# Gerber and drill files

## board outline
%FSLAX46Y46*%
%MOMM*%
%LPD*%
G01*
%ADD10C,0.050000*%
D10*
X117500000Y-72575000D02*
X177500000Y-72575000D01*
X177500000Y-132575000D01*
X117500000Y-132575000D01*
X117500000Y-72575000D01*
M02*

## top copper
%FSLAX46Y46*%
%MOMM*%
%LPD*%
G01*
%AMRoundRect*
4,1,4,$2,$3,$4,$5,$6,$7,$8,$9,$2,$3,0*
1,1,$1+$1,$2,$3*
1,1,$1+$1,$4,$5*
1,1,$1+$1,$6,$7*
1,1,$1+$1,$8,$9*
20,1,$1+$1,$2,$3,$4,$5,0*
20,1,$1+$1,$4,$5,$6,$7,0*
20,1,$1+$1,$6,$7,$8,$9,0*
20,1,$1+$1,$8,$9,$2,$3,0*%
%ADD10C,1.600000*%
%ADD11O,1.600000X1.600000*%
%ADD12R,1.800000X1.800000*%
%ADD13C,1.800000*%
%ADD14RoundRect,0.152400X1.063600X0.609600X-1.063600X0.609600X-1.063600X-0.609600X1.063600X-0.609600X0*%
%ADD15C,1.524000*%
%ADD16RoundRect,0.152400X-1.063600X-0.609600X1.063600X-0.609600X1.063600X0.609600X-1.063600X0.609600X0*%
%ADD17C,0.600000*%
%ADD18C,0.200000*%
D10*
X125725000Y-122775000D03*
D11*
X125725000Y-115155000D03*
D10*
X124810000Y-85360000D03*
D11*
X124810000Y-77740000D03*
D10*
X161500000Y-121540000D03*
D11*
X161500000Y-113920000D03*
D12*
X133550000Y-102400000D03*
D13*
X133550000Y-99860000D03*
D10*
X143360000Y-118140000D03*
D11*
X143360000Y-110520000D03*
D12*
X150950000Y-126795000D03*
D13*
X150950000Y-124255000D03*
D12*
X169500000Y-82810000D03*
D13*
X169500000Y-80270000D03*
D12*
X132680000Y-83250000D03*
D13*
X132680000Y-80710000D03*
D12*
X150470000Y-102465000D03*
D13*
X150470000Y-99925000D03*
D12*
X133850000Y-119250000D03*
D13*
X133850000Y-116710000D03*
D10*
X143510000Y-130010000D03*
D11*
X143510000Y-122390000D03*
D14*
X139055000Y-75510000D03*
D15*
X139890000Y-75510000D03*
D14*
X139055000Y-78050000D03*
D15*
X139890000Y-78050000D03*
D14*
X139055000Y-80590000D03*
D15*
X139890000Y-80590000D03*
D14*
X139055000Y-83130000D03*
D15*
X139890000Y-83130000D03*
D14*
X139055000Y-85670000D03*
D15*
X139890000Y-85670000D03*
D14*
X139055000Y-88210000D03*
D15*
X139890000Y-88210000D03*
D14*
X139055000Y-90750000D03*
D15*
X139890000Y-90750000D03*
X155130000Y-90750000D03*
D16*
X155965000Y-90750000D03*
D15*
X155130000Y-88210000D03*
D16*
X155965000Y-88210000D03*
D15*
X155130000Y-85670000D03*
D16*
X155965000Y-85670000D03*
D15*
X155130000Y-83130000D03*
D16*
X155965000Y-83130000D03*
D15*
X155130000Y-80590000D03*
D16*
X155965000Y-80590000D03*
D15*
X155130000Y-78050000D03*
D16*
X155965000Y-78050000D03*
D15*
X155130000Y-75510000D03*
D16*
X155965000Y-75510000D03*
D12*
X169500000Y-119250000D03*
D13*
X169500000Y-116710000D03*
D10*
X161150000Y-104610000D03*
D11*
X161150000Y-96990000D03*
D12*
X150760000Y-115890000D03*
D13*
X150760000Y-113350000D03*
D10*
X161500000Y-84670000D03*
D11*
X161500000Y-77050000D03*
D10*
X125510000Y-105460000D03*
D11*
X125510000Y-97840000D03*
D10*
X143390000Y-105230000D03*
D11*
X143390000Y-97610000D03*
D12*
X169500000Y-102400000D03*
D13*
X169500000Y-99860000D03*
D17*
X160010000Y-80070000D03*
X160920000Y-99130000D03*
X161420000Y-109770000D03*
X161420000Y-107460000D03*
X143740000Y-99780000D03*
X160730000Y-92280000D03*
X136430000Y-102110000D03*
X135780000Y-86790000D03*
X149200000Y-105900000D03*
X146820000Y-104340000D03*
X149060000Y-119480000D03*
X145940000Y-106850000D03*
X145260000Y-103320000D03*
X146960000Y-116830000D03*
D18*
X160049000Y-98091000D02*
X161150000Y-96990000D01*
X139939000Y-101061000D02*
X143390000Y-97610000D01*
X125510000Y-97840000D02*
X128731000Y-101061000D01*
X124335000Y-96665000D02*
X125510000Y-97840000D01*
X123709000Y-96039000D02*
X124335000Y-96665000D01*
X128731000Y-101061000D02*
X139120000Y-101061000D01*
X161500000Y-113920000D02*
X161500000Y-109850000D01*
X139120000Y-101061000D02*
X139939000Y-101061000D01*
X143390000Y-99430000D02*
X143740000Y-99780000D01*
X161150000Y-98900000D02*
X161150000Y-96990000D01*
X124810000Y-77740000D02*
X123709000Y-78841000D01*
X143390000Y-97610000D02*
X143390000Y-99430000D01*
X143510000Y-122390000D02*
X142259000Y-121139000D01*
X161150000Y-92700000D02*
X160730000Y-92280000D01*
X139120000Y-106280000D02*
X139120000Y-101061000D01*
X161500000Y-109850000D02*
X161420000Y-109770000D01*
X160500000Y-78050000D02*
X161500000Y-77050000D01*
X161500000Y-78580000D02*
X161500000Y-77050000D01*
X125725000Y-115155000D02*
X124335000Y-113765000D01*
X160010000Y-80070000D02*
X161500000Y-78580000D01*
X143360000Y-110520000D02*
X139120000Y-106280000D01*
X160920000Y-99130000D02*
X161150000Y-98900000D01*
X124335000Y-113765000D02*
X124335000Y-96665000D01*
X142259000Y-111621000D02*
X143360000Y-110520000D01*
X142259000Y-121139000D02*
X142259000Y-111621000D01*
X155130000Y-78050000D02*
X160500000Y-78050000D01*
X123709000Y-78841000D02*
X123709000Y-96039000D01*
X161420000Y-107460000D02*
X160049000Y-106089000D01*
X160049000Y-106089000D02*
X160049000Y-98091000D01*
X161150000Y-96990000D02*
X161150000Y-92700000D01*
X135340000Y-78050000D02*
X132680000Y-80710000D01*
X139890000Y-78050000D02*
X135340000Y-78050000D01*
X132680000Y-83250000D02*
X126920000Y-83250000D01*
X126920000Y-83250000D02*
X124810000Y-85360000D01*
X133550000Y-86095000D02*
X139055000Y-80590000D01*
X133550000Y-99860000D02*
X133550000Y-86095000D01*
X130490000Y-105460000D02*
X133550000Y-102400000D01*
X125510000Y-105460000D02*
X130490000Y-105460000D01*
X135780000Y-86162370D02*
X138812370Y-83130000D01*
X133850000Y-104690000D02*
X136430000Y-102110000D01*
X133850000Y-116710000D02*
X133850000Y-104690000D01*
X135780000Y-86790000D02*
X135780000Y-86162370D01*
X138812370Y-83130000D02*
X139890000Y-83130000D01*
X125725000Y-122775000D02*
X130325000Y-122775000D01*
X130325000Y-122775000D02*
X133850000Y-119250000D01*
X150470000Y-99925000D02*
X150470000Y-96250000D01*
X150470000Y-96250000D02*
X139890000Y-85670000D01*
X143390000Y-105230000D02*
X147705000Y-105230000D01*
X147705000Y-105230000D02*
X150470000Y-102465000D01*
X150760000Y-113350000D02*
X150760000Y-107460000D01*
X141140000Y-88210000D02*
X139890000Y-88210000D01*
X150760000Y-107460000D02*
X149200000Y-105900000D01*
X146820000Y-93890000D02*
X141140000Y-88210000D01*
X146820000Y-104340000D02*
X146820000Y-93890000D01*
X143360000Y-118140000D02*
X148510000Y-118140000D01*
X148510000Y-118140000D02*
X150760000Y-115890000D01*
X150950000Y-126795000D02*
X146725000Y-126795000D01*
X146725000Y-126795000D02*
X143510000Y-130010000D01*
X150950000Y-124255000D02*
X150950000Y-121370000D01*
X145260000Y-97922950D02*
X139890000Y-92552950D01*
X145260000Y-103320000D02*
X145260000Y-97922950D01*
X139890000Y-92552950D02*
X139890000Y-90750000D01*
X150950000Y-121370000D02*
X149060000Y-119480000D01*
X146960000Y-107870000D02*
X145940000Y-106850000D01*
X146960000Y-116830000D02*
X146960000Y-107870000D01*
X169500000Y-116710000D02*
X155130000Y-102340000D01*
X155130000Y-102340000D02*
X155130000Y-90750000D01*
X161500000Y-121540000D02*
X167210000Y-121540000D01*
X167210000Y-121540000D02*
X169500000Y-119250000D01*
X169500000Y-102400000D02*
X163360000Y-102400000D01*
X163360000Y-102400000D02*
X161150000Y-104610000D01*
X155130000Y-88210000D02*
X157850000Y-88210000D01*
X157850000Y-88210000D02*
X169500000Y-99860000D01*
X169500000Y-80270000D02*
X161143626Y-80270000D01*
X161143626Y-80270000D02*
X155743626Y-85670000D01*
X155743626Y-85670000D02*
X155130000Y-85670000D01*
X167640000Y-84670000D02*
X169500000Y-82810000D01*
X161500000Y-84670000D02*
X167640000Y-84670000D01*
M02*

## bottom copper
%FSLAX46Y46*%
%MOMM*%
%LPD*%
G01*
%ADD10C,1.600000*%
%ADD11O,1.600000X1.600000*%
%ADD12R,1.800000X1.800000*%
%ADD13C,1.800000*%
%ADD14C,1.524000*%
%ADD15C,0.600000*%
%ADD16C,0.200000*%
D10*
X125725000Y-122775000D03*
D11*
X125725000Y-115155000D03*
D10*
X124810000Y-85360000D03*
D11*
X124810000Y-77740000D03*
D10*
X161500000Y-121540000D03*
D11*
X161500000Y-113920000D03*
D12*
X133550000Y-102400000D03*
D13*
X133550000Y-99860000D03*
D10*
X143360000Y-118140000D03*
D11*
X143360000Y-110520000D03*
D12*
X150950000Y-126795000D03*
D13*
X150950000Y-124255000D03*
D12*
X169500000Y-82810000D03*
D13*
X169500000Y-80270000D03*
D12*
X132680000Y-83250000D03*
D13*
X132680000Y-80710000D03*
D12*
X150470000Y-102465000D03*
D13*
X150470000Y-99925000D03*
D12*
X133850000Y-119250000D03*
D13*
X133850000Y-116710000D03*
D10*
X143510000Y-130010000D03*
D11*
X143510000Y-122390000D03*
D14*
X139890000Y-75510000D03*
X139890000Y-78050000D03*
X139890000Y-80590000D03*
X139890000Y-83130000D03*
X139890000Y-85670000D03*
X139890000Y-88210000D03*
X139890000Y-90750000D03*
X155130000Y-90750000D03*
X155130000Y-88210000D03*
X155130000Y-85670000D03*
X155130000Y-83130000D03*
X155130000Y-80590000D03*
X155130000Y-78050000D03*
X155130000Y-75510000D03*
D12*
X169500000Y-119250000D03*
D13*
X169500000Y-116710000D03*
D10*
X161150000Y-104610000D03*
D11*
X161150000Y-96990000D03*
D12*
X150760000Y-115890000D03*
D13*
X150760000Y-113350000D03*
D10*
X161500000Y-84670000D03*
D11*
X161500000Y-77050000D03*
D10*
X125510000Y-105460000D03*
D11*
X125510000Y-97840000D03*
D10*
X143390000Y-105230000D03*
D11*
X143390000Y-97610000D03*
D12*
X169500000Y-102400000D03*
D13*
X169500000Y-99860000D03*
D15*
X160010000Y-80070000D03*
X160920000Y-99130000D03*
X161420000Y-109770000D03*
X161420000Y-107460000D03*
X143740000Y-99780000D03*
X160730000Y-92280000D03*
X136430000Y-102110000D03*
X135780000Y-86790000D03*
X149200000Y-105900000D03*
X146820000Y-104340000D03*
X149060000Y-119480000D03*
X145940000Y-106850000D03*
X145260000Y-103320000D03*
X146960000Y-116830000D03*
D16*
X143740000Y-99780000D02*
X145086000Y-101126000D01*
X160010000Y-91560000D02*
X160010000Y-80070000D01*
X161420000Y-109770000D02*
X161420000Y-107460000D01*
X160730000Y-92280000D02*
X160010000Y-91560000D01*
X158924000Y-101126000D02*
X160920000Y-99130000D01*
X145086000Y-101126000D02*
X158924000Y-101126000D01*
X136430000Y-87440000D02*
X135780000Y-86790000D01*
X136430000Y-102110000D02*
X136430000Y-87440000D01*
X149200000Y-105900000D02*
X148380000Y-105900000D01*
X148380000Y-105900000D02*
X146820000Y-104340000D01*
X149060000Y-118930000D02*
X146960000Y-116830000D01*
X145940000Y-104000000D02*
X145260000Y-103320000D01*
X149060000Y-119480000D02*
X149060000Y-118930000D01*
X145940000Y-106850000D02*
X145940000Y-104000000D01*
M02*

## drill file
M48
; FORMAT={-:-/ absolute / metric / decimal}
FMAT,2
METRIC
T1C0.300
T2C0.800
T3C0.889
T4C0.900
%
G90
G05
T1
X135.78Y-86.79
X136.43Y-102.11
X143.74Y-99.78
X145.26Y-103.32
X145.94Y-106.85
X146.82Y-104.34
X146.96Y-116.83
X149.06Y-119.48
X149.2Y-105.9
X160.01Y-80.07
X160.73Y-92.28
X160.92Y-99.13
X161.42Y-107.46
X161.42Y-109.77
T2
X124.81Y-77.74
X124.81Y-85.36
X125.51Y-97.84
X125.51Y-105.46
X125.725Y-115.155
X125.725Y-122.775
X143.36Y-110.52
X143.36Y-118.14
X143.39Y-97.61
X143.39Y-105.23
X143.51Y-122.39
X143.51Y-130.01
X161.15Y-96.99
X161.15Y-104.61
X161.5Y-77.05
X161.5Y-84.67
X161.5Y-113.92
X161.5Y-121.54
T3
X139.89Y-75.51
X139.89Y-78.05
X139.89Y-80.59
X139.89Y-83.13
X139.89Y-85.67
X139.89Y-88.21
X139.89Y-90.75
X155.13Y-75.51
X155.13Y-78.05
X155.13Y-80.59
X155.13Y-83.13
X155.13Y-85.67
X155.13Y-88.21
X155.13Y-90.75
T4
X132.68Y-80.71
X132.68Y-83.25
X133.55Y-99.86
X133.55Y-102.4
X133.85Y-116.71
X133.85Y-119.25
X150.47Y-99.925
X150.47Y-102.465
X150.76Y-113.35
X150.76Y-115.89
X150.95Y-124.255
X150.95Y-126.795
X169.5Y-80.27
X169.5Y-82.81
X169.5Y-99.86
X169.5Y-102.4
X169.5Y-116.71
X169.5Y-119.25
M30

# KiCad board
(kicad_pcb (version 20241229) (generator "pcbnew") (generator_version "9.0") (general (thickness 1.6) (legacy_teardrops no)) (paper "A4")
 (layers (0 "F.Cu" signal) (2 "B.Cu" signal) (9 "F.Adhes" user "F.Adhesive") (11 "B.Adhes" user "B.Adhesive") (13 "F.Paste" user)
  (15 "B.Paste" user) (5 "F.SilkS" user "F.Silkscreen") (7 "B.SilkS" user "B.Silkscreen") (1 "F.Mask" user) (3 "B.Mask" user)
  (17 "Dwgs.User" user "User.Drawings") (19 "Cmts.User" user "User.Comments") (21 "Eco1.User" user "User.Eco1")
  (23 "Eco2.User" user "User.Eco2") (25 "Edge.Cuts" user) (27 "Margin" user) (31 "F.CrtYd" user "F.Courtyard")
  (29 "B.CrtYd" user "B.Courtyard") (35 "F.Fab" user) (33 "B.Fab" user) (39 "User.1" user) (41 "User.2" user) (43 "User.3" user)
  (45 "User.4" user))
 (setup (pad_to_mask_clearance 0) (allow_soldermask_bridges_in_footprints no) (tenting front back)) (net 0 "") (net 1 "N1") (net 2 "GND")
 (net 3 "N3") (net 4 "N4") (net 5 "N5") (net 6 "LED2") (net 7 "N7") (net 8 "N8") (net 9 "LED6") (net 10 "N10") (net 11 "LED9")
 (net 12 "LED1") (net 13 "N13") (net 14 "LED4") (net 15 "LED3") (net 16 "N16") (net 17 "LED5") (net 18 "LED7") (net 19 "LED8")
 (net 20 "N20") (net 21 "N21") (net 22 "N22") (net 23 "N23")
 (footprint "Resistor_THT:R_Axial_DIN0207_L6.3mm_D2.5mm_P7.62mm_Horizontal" (layer "F.Cu") (at 125.725 122.775 90)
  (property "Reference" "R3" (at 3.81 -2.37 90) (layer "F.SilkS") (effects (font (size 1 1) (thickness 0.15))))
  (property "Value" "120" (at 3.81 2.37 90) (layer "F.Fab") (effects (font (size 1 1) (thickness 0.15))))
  (pad "1" thru_hole circle (at 0 0 90) (size 1.6 1.6) (drill 0.8) (layers "*.Cu" "*.Mask") (remove_unused_layers no) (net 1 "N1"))
  (pad "2" thru_hole oval (at 7.62 0 90) (size 1.6 1.6) (drill 0.8) (layers "*.Cu" "*.Mask") (remove_unused_layers no) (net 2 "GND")))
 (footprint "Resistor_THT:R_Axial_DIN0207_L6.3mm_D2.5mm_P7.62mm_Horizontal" (layer "F.Cu") (at 124.81 85.36 90)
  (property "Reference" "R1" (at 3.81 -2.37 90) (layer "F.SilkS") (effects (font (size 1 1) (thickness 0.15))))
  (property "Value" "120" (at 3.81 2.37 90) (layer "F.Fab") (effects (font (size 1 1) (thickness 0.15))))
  (pad "1" thru_hole circle (at 0 0 90) (size 1.6 1.6) (drill 0.8) (layers "*.Cu" "*.Mask") (remove_unused_layers no) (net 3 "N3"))
  (pad "2" thru_hole oval (at 7.62 0 90) (size 1.6 1.6) (drill 0.8) (layers "*.Cu" "*.Mask") (remove_unused_layers no) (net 2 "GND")))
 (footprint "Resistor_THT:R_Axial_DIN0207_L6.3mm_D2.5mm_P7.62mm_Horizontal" (layer "F.Cu") (at 161.5 121.54 90)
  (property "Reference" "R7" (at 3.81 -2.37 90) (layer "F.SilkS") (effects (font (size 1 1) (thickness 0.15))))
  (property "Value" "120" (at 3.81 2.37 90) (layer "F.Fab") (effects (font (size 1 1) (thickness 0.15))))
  (pad "1" thru_hole circle (at 0 0 90) (size 1.6 1.6) (drill 0.8) (layers "*.Cu" "*.Mask") (remove_unused_layers no) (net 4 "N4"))
  (pad "2" thru_hole oval (at 7.62 0 90) (size 1.6 1.6) (drill 0.8) (layers "*.Cu" "*.Mask") (remove_unused_layers no) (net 2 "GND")))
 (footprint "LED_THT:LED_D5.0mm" (layer "F.Cu") (at 133.55 102.4 90)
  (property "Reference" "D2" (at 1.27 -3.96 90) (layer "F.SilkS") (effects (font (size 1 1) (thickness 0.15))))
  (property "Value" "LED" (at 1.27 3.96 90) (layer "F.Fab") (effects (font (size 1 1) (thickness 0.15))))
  (pad "1" thru_hole rect (at 0 0 90) (size 1.8 1.8) (drill 0.9) (layers "*.Cu" "*.Mask") (remove_unused_layers no) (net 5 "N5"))
  (pad "2" thru_hole circle (at 2.54 0 90) (size 1.8 1.8) (drill 0.9) (layers "*.Cu" "*.Mask") (remove_unused_layers no) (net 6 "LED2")))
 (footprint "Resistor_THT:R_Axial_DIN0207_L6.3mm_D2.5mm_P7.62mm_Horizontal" (layer "F.Cu") (at 143.36 118.14 90)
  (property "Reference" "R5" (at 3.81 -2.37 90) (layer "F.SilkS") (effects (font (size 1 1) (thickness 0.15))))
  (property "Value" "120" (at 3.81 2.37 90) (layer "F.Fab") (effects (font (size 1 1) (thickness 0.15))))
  (pad "1" thru_hole circle (at 0 0 90) (size 1.6 1.6) (drill 0.8) (layers "*.Cu" "*.Mask") (remove_unused_layers no) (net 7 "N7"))
  (pad "2" thru_hole oval (at 7.62 0 90) (size 1.6 1.6) (drill 0.8) (layers "*.Cu" "*.Mask") (remove_unused_layers no) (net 2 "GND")))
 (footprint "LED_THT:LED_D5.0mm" (layer "F.Cu") (at 150.95 126.795 90)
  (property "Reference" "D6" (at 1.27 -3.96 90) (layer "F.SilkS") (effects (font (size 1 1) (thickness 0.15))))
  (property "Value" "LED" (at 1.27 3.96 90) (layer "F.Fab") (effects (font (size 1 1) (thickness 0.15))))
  (pad "1" thru_hole rect (at 0 0 90) (size 1.8 1.8) (drill 0.9) (layers "*.Cu" "*.Mask") (remove_unused_layers no) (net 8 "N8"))
  (pad "2" thru_hole circle (at 2.54 0 90) (size 1.8 1.8) (drill 0.9) (layers "*.Cu" "*.Mask") (remove_unused_layers no) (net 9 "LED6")))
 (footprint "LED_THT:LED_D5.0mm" (layer "F.Cu") (at 169.5 82.81 90)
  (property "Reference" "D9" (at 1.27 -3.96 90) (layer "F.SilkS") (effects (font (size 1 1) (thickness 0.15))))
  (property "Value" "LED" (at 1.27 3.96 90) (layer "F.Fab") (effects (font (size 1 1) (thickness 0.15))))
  (pad "1" thru_hole rect (at 0 0 90) (size 1.8 1.8) (drill 0.9) (layers "*.Cu" "*.Mask") (remove_unused_layers no) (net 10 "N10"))
  (pad "2" thru_hole circle (at 2.54 0 90) (size 1.8 1.8) (drill 0.9) (layers "*.Cu" "*.Mask") (remove_unused_layers no) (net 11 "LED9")))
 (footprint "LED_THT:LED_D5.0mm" (layer "F.Cu") (at 132.68 83.25 90)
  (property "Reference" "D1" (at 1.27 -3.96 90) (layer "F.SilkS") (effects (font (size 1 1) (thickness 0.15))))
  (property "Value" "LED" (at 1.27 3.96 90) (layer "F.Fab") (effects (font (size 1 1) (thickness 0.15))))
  (pad "1" thru_hole rect (at 0 0 90) (size 1.8 1.8) (drill 0.9) (layers "*.Cu" "*.Mask") (remove_unused_layers no) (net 3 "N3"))
  (pad "2" thru_hole circle (at 2.54 0 90) (size 1.8 1.8) (drill 0.9) (layers "*.Cu" "*.Mask") (remove_unused_layers no) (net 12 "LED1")))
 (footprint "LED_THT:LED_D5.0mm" (layer "F.Cu") (at 150.47 102.465 90)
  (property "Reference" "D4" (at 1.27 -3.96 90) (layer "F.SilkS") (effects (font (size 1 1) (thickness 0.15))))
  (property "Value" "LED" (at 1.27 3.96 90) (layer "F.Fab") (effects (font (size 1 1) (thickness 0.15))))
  (pad "1" thru_hole rect (at 0 0 90) (size 1.8 1.8) (drill 0.9) (layers "*.Cu" "*.Mask") (remove_unused_layers no) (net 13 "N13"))
  (pad "2" thru_hole circle (at 2.54 0 90) (size 1.8 1.8) (drill 0.9) (layers "*.Cu" "*.Mask") (remove_unused_layers no) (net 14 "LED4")))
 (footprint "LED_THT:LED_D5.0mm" (layer "F.Cu") (at 133.85 119.25 90)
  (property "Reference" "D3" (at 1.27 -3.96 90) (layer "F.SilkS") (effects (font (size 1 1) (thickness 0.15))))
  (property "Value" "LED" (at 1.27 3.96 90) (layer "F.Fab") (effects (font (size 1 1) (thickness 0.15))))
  (pad "1" thru_hole rect (at 0 0 90) (size 1.8 1.8) (drill 0.9) (layers "*.Cu" "*.Mask") (remove_unused_layers no) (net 1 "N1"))
  (pad "2" thru_hole circle (at 2.54 0 90) (size 1.8 1.8) (drill 0.9) (layers "*.Cu" "*.Mask") (remove_unused_layers no) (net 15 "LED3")))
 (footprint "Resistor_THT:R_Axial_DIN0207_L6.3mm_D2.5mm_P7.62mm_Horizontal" (layer "F.Cu") (at 143.51 130.01 90)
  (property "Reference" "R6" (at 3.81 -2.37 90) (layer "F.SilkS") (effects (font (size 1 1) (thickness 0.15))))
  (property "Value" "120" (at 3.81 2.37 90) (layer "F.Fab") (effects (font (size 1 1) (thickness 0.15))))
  (pad "1" thru_hole circle (at 0 0 90) (size 1.6 1.6) (drill 0.8) (layers "*.Cu" "*.Mask") (remove_unused_layers no) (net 8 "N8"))
  (pad "2" thru_hole oval (at 7.62 0 90) (size 1.6 1.6) (drill 0.8) (layers "*.Cu" "*.Mask") (remove_unused_layers no) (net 2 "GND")))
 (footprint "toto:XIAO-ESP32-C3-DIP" (layer "F.Cu") (at 147.51 83.13 90)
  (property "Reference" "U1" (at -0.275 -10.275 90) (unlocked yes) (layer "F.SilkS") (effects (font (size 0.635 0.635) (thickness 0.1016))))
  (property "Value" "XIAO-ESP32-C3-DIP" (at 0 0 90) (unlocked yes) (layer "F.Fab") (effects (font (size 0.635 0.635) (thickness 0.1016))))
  (pad "1" smd roundrect (at 7.62 -8.455 180) (size 2.432 1.524) (layers "F.Cu" "F.Mask") (roundrect_rratio 0.1) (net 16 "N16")
   (thermal_bridge_angle 45))
  (pad "1" thru_hole circle (at 7.62 -7.62 180) (size 1.524 1.524) (drill 0.889) (layers "*.Cu" "*.Mask") (remove_unused_layers no)
   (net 16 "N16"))
  (pad "2" smd roundrect (at 5.08 -8.455 180) (size 2.432 1.524) (layers "F.Cu" "F.Mask") (roundrect_rratio 0.1) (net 12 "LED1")
   (thermal_bridge_angle 45))
  (pad "2" thru_hole circle (at 5.08 -7.62 180) (size 1.524 1.524) (drill 0.889) (layers "*.Cu" "*.Mask") (remove_unused_layers no)
   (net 12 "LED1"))
  (pad "3" smd roundrect (at 2.54 -8.455 180) (size 2.432 1.524) (layers "F.Cu" "F.Mask") (roundrect_rratio 0.1) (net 6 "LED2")
   (thermal_bridge_angle 45))
  (pad "3" thru_hole circle (at 2.54 -7.62 180) (size 1.524 1.524) (drill 0.889) (layers "*.Cu" "*.Mask") (remove_unused_layers no)
   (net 6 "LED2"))
  (pad "4" smd roundrect (at 0 -8.455 180) (size 2.432 1.524) (layers "F.Cu" "F.Mask") (roundrect_rratio 0.1) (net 15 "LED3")
   (thermal_bridge_angle 45))
  (pad "4" thru_hole circle (at 0 -7.62 180) (size 1.524 1.524) (drill 0.889) (layers "*.Cu" "*.Mask") (remove_unused_layers no)
   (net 15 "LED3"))
  (pad "5" smd roundrect (at -2.54 -8.455 180) (size 2.432 1.524) (layers "F.Cu" "F.Mask") (roundrect_rratio 0.1) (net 14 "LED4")
   (thermal_bridge_angle 45))
  (pad "5" thru_hole circle (at -2.54 -7.62 180) (size 1.524 1.524) (drill 0.889) (layers "*.Cu" "*.Mask") (remove_unused_layers no)
   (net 14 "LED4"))
  (pad "6" smd roundrect (at -5.08 -8.455 180) (size 2.432 1.524) (layers "F.Cu" "F.Mask") (roundrect_rratio 0.1) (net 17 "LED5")
   (thermal_bridge_angle 45))
  (pad "6" thru_hole circle (at -5.08 -7.62 180) (size 1.524 1.524) (drill 0.889) (layers "*.Cu" "*.Mask") (remove_unused_layers no)
   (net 17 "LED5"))
  (pad "7" smd roundrect (at -7.62 -8.455 180) (size 2.432 1.524) (layers "F.Cu" "F.Mask") (roundrect_rratio 0.1) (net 9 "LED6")
   (thermal_bridge_angle 45))
  (pad "7" thru_hole circle (at -7.62 -7.62 180) (size 1.524 1.524) (drill 0.889) (layers "*.Cu" "*.Mask") (remove_unused_layers no)
   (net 9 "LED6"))
  (pad "8" thru_hole circle (at -7.62 7.62) (size 1.524 1.524) (drill 0.889) (layers "*.Cu" "*.Mask") (remove_unused_layers no)
   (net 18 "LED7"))
  (pad "8" smd roundrect (at -7.62 8.455) (size 2.432 1.524) (layers "F.Cu" "F.Mask") (roundrect_rratio 0.1) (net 18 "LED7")
   (thermal_bridge_angle 45))
  (pad "9" thru_hole circle (at -5.08 7.62) (size 1.524 1.524) (drill 0.889) (layers "*.Cu" "*.Mask") (remove_unused_layers no)
   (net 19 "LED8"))
  (pad "9" smd roundrect (at -5.08 8.455) (size 2.432 1.524) (layers "F.Cu" "F.Mask") (roundrect_rratio 0.1) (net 19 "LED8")
   (thermal_bridge_angle 45))
  (pad "10" thru_hole circle (at -2.54 7.62) (size 1.524 1.524) (drill 0.889) (layers "*.Cu" "*.Mask") (remove_unused_layers no)
   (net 11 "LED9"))
  (pad "10" smd roundrect (at -2.54 8.455) (size 2.432 1.524) (layers "F.Cu" "F.Mask") (roundrect_rratio 0.1) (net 11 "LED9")
   (thermal_bridge_angle 45))
  (pad "11" thru_hole circle (at 0 7.62) (size 1.524 1.524) (drill 0.889) (layers "*.Cu" "*.Mask") (remove_unused_layers no) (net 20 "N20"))
  (pad "11" smd roundrect (at 0 8.455) (size 2.432 1.524) (layers "F.Cu" "F.Mask") (roundrect_rratio 0.1) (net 20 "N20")
   (thermal_bridge_angle 45))
  (pad "12" thru_hole circle (at 2.54 7.62) (size 1.524 1.524) (drill 0.889) (layers "*.Cu" "*.Mask") (remove_unused_layers no)
   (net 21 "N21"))
  (pad "12" smd roundrect (at 2.54 8.455) (size 2.432 1.524) (layers "F.Cu" "F.Mask") (roundrect_rratio 0.1) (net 21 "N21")
   (thermal_bridge_angle 45))
  (pad "13" thru_hole circle (at 5.08 7.62) (size 1.524 1.524) (drill 0.889) (layers "*.Cu" "*.Mask") (remove_unused_layers no)
   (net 2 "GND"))
  (pad "13" smd roundrect (at 5.08 8.455) (size 2.432 1.524) (layers "F.Cu" "F.Mask") (roundrect_rratio 0.1) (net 2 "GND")
   (thermal_bridge_angle 45))
  (pad "14" thru_hole circle (at 7.62 7.62) (size 1.524 1.524) (drill 0.889) (layers "*.Cu" "*.Mask") (remove_unused_layers no)
   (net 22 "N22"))
  (pad "14" smd roundrect (at 7.62 8.455) (size 2.432 1.524) (layers "F.Cu" "F.Mask") (roundrect_rratio 0.1) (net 22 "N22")
   (thermal_bridge_angle 45)))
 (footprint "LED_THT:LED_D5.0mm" (layer "F.Cu") (at 169.5 119.25 90)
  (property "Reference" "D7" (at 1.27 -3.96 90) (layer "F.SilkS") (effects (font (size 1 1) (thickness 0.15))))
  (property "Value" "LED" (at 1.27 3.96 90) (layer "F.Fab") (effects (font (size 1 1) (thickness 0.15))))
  (pad "1" thru_hole rect (at 0 0 90) (size 1.8 1.8) (drill 0.9) (layers "*.Cu" "*.Mask") (remove_unused_layers no) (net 4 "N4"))
  (pad "2" thru_hole circle (at 2.54 0 90) (size 1.8 1.8) (drill 0.9) (layers "*.Cu" "*.Mask") (remove_unused_layers no) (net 18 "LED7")))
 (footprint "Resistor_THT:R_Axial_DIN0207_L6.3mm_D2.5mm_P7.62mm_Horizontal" (layer "F.Cu") (at 161.15 104.61 90)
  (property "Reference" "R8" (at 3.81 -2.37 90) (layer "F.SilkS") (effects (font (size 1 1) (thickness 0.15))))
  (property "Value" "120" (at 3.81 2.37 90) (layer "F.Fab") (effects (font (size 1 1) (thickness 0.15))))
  (pad "1" thru_hole circle (at 0 0 90) (size 1.6 1.6) (drill 0.8) (layers "*.Cu" "*.Mask") (remove_unused_layers no) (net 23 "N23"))
  (pad "2" thru_hole oval (at 7.62 0 90) (size 1.6 1.6) (drill 0.8) (layers "*.Cu" "*.Mask") (remove_unused_layers no) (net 2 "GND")))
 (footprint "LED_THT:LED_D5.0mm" (layer "F.Cu") (at 150.76 115.89 90)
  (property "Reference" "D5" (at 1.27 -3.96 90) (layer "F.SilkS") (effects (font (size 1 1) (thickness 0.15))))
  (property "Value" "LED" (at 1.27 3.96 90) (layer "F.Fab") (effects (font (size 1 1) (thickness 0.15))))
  (pad "1" thru_hole rect (at 0 0 90) (size 1.8 1.8) (drill 0.9) (layers "*.Cu" "*.Mask") (remove_unused_layers no) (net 7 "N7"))
  (pad "2" thru_hole circle (at 2.54 0 90) (size 1.8 1.8) (drill 0.9) (layers "*.Cu" "*.Mask") (remove_unused_layers no) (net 17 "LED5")))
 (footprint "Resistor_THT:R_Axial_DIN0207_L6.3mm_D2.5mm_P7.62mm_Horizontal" (layer "F.Cu") (at 161.5 84.67 90)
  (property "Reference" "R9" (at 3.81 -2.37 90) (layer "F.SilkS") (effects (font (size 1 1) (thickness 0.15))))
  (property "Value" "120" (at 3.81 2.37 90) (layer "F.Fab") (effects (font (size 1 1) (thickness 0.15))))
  (pad "1" thru_hole circle (at 0 0 90) (size 1.6 1.6) (drill 0.8) (layers "*.Cu" "*.Mask") (remove_unused_layers no) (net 10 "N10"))
  (pad "2" thru_hole oval (at 7.62 0 90) (size 1.6 1.6) (drill 0.8) (layers "*.Cu" "*.Mask") (remove_unused_layers no) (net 2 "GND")))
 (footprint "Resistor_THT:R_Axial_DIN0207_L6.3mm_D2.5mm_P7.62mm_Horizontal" (layer "F.Cu") (at 125.51 105.46 90)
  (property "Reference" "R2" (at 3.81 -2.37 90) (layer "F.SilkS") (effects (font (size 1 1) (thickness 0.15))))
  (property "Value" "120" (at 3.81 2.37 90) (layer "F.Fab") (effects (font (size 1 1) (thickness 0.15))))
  (pad "1" thru_hole circle (at 0 0 90) (size 1.6 1.6) (drill 0.8) (layers "*.Cu" "*.Mask") (remove_unused_layers no) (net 5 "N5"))
  (pad "2" thru_hole oval (at 7.62 0 90) (size 1.6 1.6) (drill 0.8) (layers "*.Cu" "*.Mask") (remove_unused_layers no) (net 2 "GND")))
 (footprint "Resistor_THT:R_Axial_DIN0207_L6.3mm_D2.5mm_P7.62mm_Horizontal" (layer "F.Cu") (at 143.39 105.23 90)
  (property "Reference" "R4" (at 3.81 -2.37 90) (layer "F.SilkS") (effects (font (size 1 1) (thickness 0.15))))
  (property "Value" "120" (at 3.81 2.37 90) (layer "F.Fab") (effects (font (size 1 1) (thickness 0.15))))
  (pad "1" thru_hole circle (at 0 0 90) (size 1.6 1.6) (drill 0.8) (layers "*.Cu" "*.Mask") (remove_unused_layers no) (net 13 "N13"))
  (pad "2" thru_hole oval (at 7.62 0 90) (size 1.6 1.6) (drill 0.8) (layers "*.Cu" "*.Mask") (remove_unused_layers no) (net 2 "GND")))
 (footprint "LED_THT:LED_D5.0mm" (layer "F.Cu") (at 169.5 102.4 90)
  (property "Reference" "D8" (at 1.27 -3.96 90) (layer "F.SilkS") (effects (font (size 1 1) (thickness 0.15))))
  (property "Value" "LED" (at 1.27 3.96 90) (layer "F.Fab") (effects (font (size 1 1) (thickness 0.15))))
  (pad "1" thru_hole rect (at 0 0 90) (size 1.8 1.8) (drill 0.9) (layers "*.Cu" "*.Mask") (remove_unused_layers no) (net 23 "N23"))
  (pad "2" thru_hole circle (at 2.54 0 90) (size 1.8 1.8) (drill 0.9) (layers "*.Cu" "*.Mask") (remove_unused_layers no) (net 19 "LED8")))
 (gr_rect (start 117.5 72.575) (end 177.5 132.575) (stroke (width 0.05) (type default)) (fill no) (layer "Edge.Cuts"))
 (segment (start 160.049 98.091) (end 161.15 96.99) (width 0.2) (layer "F.Cu") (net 2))
 (segment (start 139.939 101.061) (end 143.39 97.61) (width 0.2) (layer "F.Cu") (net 2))
 (segment (start 125.51 97.84) (end 128.731 101.061) (width 0.2) (layer "F.Cu") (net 2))
 (segment (start 124.335 96.665) (end 125.51 97.84) (width 0.2) (layer "F.Cu") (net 2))
 (segment (start 123.709 96.039) (end 124.335 96.665) (width 0.2) (layer "F.Cu") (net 2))
 (segment (start 128.731 101.061) (end 139.12 101.061) (width 0.2) (layer "F.Cu") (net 2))
 (segment (start 161.5 113.92) (end 161.5 109.85) (width 0.2) (layer "F.Cu") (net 2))
 (segment (start 139.12 101.061) (end 139.939 101.061) (width 0.2) (layer "F.Cu") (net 2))
 (segment (start 143.39 99.43) (end 143.74 99.78) (width 0.2) (layer "F.Cu") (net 2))
 (segment (start 161.15 98.9) (end 161.15 96.99) (width 0.2) (layer "F.Cu") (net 2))
 (segment (start 124.81 77.74) (end 123.709 78.841) (width 0.2) (layer "F.Cu") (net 2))
 (segment (start 143.39 97.61) (end 143.39 99.43) (width 0.2) (layer "F.Cu") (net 2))
 (segment (start 143.51 122.39) (end 142.259 121.139) (width 0.2) (layer "F.Cu") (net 2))
 (segment (start 161.15 92.7) (end 160.73 92.28) (width 0.2) (layer "F.Cu") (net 2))
 (segment (start 139.12 106.28) (end 139.12 101.061) (width 0.2) (layer "F.Cu") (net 2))
 (segment (start 161.5 109.85) (end 161.42 109.77) (width 0.2) (layer "F.Cu") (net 2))
 (segment (start 160.5 78.05) (end 161.5 77.05) (width 0.2) (layer "F.Cu") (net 2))
 (segment (start 161.5 78.58) (end 161.5 77.05) (width 0.2) (layer "F.Cu") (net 2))
 (segment (start 125.725 115.155) (end 124.335 113.765) (width 0.2) (layer "F.Cu") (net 2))
 (segment (start 160.01 80.07) (end 161.5 78.58) (width 0.2) (layer "F.Cu") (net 2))
 (segment (start 143.36 110.52) (end 139.12 106.28) (width 0.2) (layer "F.Cu") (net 2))
 (segment (start 160.92 99.13) (end 161.15 98.9) (width 0.2) (layer "F.Cu") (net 2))
 (segment (start 124.335 113.765) (end 124.335 96.665) (width 0.2) (layer "F.Cu") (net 2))
 (segment (start 142.259 111.621) (end 143.36 110.52) (width 0.2) (layer "F.Cu") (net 2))
 (segment (start 142.259 121.139) (end 142.259 111.621) (width 0.2) (layer "F.Cu") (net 2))
 (segment (start 155.13 78.05) (end 160.5 78.05) (width 0.2) (layer "F.Cu") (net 2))
 (segment (start 123.709 78.841) (end 123.709 96.039) (width 0.2) (layer "F.Cu") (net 2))
 (segment (start 161.42 107.46) (end 160.049 106.089) (width 0.2) (layer "F.Cu") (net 2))
 (segment (start 160.049 106.089) (end 160.049 98.091) (width 0.2) (layer "F.Cu") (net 2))
 (segment (start 161.15 96.99) (end 161.15 92.7) (width 0.2) (layer "F.Cu") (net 2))
 (via (at 160.01 80.07) (size 0.6) (drill 0.3) (layers "F.Cu" "B.Cu") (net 2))
 (via (at 160.92 99.13) (size 0.6) (drill 0.3) (layers "F.Cu" "B.Cu") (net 2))
 (via (at 161.42 109.77) (size 0.6) (drill 0.3) (layers "F.Cu" "B.Cu") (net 2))
 (via (at 161.42 107.46) (size 0.6) (drill 0.3) (layers "F.Cu" "B.Cu") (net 2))
 (via (at 143.74 99.78) (size 0.6) (drill 0.3) (layers "F.Cu" "B.Cu") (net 2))
 (via (at 160.73 92.28) (size 0.6) (drill 0.3) (layers "F.Cu" "B.Cu") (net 2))
 (segment (start 143.74 99.78) (end 145.086 101.126) (width 0.2) (layer "B.Cu") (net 2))
 (segment (start 160.01 91.56) (end 160.01 80.07) (width 0.2) (layer "B.Cu") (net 2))
 (segment (start 161.42 109.77) (end 161.42 107.46) (width 0.2) (layer "B.Cu") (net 2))
 (segment (start 160.73 92.28) (end 160.01 91.56) (width 0.2) (layer "B.Cu") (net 2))
 (segment (start 158.924 101.126) (end 160.92 99.13) (width 0.2) (layer "B.Cu") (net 2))
 (segment (start 145.086 101.126) (end 158.924 101.126) (width 0.2) (layer "B.Cu") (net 2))
 (segment (start 135.34 78.05) (end 132.68 80.71) (width 0.2) (layer "F.Cu") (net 12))
 (segment (start 139.89 78.05) (end 135.34 78.05) (width 0.2) (layer "F.Cu") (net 12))
 (segment (start 132.68 83.25) (end 126.92 83.25) (width 0.2) (layer "F.Cu") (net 3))
 (segment (start 126.92 83.25) (end 124.81 85.36) (width 0.2) (layer "F.Cu") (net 3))
 (segment (start 133.55 86.095) (end 139.055 80.59) (width 0.2) (layer "F.Cu") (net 6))
 (segment (start 133.55 99.86) (end 133.55 86.095) (width 0.2) (layer "F.Cu") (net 6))
 (segment (start 130.49 105.46) (end 133.55 102.4) (width 0.2) (layer "F.Cu") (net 5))
 (segment (start 125.51 105.46) (end 130.49 105.46) (width 0.2) (layer "F.Cu") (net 5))
 (segment (start 135.78 86.16237) (end 138.81237 83.13) (width 0.2) (layer "F.Cu") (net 15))
 (segment (start 133.85 104.69) (end 136.43 102.11) (width 0.2) (layer "F.Cu") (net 15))
 (segment (start 133.85 116.71) (end 133.85 104.69) (width 0.2) (layer "F.Cu") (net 15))
 (segment (start 135.78 86.79) (end 135.78 86.16237) (width 0.2) (layer "F.Cu") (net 15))
 (segment (start 138.81237 83.13) (end 139.89 83.13) (width 0.2) (layer "F.Cu") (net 15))
 (via (at 136.43 102.11) (size 0.6) (drill 0.3) (layers "F.Cu" "B.Cu") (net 15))
 (via (at 135.78 86.79) (size 0.6) (drill 0.3) (layers "F.Cu" "B.Cu") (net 15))
 (segment (start 136.43 87.44) (end 135.78 86.79) (width 0.2) (layer "B.Cu") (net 15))
 (segment (start 136.43 102.11) (end 136.43 87.44) (width 0.2) (layer "B.Cu") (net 15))
 (segment (start 125.725 122.775) (end 130.325 122.775) (width 0.2) (layer "F.Cu") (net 1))
 (segment (start 130.325 122.775) (end 133.85 119.25) (width 0.2) (layer "F.Cu") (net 1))
 (segment (start 150.47 99.925) (end 150.47 96.25) (width 0.2) (layer "F.Cu") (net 14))
 (segment (start 150.47 96.25) (end 139.89 85.67) (width 0.2) (layer "F.Cu") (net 14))
 (segment (start 143.39 105.23) (end 147.705 105.23) (width 0.2) (layer "F.Cu") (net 13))
 (segment (start 147.705 105.23) (end 150.47 102.465) (width 0.2) (layer "F.Cu") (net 13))
 (segment (start 150.76 113.35) (end 150.76 107.46) (width 0.2) (layer "F.Cu") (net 17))
 (segment (start 141.14 88.21) (end 139.89 88.21) (width 0.2) (layer "F.Cu") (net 17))
 (segment (start 150.76 107.46) (end 149.2 105.9) (width 0.2) (layer "F.Cu") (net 17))
 (segment (start 146.82 93.89) (end 141.14 88.21) (width 0.2) (layer "F.Cu") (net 17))
 (segment (start 146.82 104.34) (end 146.82 93.89) (width 0.2) (layer "F.Cu") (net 17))
 (via (at 149.2 105.9) (size 0.6) (drill 0.3) (layers "F.Cu" "B.Cu") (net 17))
 (via (at 146.82 104.34) (size 0.6) (drill 0.3) (layers "F.Cu" "B.Cu") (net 17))
 (segment (start 149.2 105.9) (end 148.38 105.9) (width 0.2) (layer "B.Cu") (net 17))
 (segment (start 148.38 105.9) (end 146.82 104.34) (width 0.2) (layer "B.Cu") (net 17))
 (segment (start 143.36 118.14) (end 148.51 118.14) (width 0.2) (layer "F.Cu") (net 7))
 (segment (start 148.51 118.14) (end 150.76 115.89) (width 0.2) (layer "F.Cu") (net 7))
 (segment (start 150.95 126.795) (end 146.725 126.795) (width 0.2) (layer "F.Cu") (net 8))
 (segment (start 146.725 126.795) (end 143.51 130.01) (width 0.2) (layer "F.Cu") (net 8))
 (segment (start 150.95 124.255) (end 150.95 121.37) (width 0.2) (layer "F.Cu") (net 9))
 (segment (start 145.26 97.92295) (end 139.89 92.55295) (width 0.2) (layer "F.Cu") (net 9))
 (segment (start 145.26 103.32) (end 145.26 97.92295) (width 0.2) (layer "F.Cu") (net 9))
 (segment (start 139.89 92.55295) (end 139.89 90.75) (width 0.2) (layer "F.Cu") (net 9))
 (segment (start 150.95 121.37) (end 149.06 119.48) (width 0.2) (layer "F.Cu") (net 9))
 (segment (start 146.96 107.87) (end 145.94 106.85) (width 0.2) (layer "F.Cu") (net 9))
 (segment (start 146.96 116.83) (end 146.96 107.87) (width 0.2) (layer "F.Cu") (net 9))
 (via (at 149.06 119.48) (size 0.6) (drill 0.3) (layers "F.Cu" "B.Cu") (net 9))
 (via (at 145.94 106.85) (size 0.6) (drill 0.3) (layers "F.Cu" "B.Cu") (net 9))
 (via (at 145.26 103.32) (size 0.6) (drill 0.3) (layers "F.Cu" "B.Cu") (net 9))
 (via (at 146.96 116.83) (size 0.6) (drill 0.3) (layers "F.Cu" "B.Cu") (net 9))
 (segment (start 149.06 118.93) (end 146.96 116.83) (width 0.2) (layer "B.Cu") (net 9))
 (segment (start 145.94 104) (end 145.26 103.32) (width 0.2) (layer "B.Cu") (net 9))
 (segment (start 149.06 119.48) (end 149.06 118.93) (width 0.2) (layer "B.Cu") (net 9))
 (segment (start 145.94 106.85) (end 145.94 104) (width 0.2) (layer "B.Cu") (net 9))
 (segment (start 169.5 116.71) (end 155.13 102.34) (width 0.2) (layer "F.Cu") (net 18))
 (segment (start 155.13 102.34) (end 155.13 90.75) (width 0.2) (layer "F.Cu") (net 18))
 (segment (start 161.5 121.54) (end 167.21 121.54) (width 0.2) (layer "F.Cu") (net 4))
 (segment (start 167.21 121.54) (end 169.5 119.25) (width 0.2) (layer "F.Cu") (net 4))
 (segment (start 169.5 102.4) (end 163.36 102.4) (width 0.2) (layer "F.Cu") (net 23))
 (segment (start 163.36 102.4) (end 161.15 104.61) (width 0.2) (layer "F.Cu") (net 23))
 (segment (start 155.13 88.21) (end 157.85 88.21) (width 0.2) (layer "F.Cu") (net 19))
 (segment (start 157.85 88.21) (end 169.5 99.86) (width 0.2) (layer "F.Cu") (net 19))
 (segment (start 169.5 80.27) (end 161.143626 80.27) (width 0.2) (layer "F.Cu") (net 11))
 (segment (start 161.143626 80.27) (end 155.743626 85.67) (width 0.2) (layer "F.Cu") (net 11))
 (segment (start 155.743626 85.67) (end 155.13 85.67) (width 0.2) (layer "F.Cu") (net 11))
 (segment (start 167.64 84.67) (end 169.5 82.81) (width 0.2) (layer "F.Cu") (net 10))
 (segment (start 161.5 84.67) (end 167.64 84.67) (width 0.2) (layer "F.Cu") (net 10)))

